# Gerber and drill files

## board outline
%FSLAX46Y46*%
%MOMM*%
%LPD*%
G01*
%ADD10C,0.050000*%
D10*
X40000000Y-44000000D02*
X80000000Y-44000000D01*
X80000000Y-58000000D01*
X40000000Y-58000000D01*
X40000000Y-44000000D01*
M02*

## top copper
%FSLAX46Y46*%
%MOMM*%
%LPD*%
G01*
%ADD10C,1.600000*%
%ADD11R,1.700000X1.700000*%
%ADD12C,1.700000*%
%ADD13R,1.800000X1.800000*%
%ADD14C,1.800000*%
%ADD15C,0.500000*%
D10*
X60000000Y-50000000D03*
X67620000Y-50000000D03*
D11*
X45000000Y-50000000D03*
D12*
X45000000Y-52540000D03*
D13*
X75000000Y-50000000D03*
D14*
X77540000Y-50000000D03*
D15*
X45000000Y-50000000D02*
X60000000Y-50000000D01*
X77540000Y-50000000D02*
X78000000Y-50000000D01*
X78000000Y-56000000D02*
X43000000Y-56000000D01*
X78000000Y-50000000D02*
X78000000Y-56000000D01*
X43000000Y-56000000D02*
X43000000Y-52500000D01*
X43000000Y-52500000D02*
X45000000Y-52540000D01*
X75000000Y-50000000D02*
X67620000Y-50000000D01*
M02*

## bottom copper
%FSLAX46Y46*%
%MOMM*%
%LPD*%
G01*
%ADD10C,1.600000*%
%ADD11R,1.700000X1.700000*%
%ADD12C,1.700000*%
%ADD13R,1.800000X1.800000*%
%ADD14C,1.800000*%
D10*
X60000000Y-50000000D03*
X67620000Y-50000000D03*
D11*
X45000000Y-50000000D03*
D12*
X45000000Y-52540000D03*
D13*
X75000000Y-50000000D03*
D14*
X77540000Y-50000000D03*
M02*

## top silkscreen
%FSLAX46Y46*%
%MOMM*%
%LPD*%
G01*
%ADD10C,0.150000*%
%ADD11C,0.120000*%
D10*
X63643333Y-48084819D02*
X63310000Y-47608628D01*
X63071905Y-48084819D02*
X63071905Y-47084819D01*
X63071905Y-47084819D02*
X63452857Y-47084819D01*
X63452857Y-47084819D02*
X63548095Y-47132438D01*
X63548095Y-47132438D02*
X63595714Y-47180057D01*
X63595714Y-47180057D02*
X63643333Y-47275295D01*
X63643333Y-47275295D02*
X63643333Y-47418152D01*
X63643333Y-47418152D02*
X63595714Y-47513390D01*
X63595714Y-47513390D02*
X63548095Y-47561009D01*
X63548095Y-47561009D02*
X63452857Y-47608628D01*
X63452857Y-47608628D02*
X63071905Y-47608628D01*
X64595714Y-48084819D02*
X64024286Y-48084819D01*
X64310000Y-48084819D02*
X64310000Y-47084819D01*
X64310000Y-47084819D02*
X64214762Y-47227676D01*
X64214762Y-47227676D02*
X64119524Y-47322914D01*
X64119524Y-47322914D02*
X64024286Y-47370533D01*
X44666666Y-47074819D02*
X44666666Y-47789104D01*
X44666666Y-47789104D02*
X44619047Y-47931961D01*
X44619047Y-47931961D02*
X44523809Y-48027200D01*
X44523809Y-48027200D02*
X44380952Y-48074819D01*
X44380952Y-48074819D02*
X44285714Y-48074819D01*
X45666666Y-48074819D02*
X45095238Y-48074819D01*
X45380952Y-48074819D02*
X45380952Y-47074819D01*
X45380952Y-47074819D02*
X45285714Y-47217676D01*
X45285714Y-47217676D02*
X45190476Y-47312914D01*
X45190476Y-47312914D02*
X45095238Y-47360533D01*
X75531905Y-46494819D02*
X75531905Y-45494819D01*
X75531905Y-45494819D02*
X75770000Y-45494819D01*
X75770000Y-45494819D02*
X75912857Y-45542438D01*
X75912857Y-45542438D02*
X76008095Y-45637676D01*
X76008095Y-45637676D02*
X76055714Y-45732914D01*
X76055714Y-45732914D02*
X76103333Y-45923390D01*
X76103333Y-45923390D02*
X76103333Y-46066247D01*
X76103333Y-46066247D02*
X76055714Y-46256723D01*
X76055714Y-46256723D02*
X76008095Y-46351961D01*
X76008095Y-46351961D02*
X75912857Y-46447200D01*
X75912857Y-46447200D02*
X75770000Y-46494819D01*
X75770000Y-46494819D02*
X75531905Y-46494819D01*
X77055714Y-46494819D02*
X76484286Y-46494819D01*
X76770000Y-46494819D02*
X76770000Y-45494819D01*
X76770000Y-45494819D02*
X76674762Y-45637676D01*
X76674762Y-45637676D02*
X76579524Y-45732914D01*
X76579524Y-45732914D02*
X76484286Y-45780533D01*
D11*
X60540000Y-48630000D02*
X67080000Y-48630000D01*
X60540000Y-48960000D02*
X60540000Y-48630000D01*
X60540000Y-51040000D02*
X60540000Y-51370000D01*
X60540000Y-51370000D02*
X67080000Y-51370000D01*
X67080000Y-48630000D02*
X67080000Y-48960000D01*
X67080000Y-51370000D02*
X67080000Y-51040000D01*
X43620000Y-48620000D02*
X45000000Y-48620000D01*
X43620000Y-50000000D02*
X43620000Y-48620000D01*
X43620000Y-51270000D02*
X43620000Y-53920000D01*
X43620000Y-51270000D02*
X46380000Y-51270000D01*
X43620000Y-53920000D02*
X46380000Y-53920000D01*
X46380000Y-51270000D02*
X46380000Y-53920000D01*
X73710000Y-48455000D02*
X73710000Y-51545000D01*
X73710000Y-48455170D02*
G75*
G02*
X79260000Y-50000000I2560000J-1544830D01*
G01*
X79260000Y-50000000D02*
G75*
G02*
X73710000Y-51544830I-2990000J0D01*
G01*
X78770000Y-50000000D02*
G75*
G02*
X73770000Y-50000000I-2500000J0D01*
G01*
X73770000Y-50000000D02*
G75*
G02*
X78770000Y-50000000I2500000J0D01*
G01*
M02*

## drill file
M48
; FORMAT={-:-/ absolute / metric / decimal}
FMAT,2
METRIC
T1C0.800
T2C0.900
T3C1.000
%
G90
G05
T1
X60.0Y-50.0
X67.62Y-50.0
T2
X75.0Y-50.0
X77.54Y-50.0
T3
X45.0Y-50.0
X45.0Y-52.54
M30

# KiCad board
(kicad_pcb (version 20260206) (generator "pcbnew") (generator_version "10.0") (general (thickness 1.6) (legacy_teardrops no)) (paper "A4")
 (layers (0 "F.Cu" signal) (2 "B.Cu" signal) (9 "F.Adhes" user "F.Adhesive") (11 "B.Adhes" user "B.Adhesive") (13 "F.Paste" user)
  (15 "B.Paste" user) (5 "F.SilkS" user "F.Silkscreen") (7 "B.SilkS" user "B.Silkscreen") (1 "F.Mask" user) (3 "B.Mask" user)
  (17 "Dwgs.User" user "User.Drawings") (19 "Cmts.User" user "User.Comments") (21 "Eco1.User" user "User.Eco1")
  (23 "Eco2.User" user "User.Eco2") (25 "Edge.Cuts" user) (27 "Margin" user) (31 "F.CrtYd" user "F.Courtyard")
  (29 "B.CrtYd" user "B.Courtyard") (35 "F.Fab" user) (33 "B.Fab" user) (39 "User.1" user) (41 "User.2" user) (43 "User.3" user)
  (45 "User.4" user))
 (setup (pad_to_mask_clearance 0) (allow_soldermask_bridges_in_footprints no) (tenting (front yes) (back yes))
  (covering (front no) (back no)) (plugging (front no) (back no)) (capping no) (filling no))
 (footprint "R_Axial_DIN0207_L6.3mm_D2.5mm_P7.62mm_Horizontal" (layer "F.Cu") (at 60 50)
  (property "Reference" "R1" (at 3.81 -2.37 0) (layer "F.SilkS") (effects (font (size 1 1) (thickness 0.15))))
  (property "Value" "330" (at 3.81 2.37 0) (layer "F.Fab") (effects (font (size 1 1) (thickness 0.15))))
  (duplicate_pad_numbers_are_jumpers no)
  (fp_line (start 0.54 -1.37) (end 7.08 -1.37) (stroke (width 0.12) (type solid)) (layer "F.SilkS"))
  (fp_line (start 0.54 -1.04) (end 0.54 -1.37) (stroke (width 0.12) (type solid)) (layer "F.SilkS"))
  (fp_line (start 0.54 1.04) (end 0.54 1.37) (stroke (width 0.12) (type solid)) (layer "F.SilkS"))
  (fp_line (start 0.54 1.37) (end 7.08 1.37) (stroke (width 0.12) (type solid)) (layer "F.SilkS"))
  (fp_line (start 7.08 -1.37) (end 7.08 -1.04) (stroke (width 0.12) (type solid)) (layer "F.SilkS"))
  (fp_line (start 7.08 1.37) (end 7.08 1.04) (stroke (width 0.12) (type solid)) (layer "F.SilkS"))
  (pad "1" thru_hole circle (at 0 0) (size 1.6 1.6) (drill 0.8) (layers "*.Cu" "*.Mask") (remove_unused_layers no) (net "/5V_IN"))
  (pad "2" thru_hole circle (at 7.62 0) (size 1.6 1.6) (drill 0.8) (layers "*.Cu" "*.Mask") (remove_unused_layers no) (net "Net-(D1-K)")))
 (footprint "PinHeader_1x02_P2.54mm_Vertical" (layer "F.Cu") (at 45 50)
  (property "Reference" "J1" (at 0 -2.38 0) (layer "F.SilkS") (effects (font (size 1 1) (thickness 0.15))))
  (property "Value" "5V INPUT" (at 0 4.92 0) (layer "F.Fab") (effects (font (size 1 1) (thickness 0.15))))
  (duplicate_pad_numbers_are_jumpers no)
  (fp_line (start -1.38 -1.38) (end 0 -1.38) (stroke (width 0.12) (type solid)) (layer "F.SilkS"))
  (fp_line (start -1.38 0) (end -1.38 -1.38) (stroke (width 0.12) (type solid)) (layer "F.SilkS"))
  (fp_line (start -1.38 1.27) (end -1.38 3.92) (stroke (width 0.12) (type solid)) (layer "F.SilkS"))
  (fp_line (start -1.38 1.27) (end 1.38 1.27) (stroke (width 0.12) (type solid)) (layer "F.SilkS"))
  (fp_line (start -1.38 3.92) (end 1.38 3.92) (stroke (width 0.12) (type solid)) (layer "F.SilkS"))
  (fp_line (start 1.38 1.27) (end 1.38 3.92) (stroke (width 0.12) (type solid)) (layer "F.SilkS"))
  (pad "1" thru_hole rect (at 0 0) (size 1.7 1.7) (drill 1) (layers "*.Cu" "*.Mask") (remove_unused_layers no) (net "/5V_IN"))
  (pad "2" thru_hole circle (at 0 2.54) (size 1.7 1.7) (drill 1) (layers "*.Cu" "*.Mask") (remove_unused_layers no) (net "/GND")))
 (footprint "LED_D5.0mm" (layer "F.Cu") (at 75 50)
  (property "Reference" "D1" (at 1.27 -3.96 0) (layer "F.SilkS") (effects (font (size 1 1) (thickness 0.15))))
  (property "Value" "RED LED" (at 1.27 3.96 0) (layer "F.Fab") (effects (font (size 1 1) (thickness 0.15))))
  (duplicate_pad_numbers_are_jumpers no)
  (fp_line (start -1.29 -1.545) (end -1.29 1.545) (stroke (width 0.12) (type solid)) (layer "F.SilkS"))
  (fp_arc (start -1.29 -1.54483) (mid 2.071779 -2.880495) (end 4.26 0) (stroke (width 0.12) (type solid)) (layer "F.SilkS"))
  (fp_arc (start 4.26 0) (mid 2.071779 2.880495) (end -1.29 1.54483) (stroke (width 0.12) (type solid)) (layer "F.SilkS"))
  (fp_circle (center 1.27 0) (end 3.77 0) (stroke (width 0.12) (type solid)) (fill no) (layer "F.SilkS"))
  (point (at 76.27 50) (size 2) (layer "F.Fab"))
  (pad "1" thru_hole rect (at 0 0) (size 1.8 1.8) (drill 0.9) (layers "*.Cu" "*.Mask") (remove_unused_layers no) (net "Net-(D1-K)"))
  (pad "2" thru_hole circle (at 2.54 0) (size 1.8 1.8) (drill 0.9) (layers "*.Cu" "*.Mask") (remove_unused_layers no) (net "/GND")))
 (gr_rect (start 40 44) (end 80 58) (stroke (width 0.05) (type default)) (fill no) (layer "Edge.Cuts"))
 (segment (start 45 50) (end 60 50) (width 0.5) (layer "F.Cu") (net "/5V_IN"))
 (segment (start 77.54 50) (end 78 50) (width 0.5) (layer "F.Cu") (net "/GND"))
 (segment (start 78 56) (end 43 56) (width 0.5) (layer "F.Cu") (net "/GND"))
 (segment (start 78 50) (end 78 56) (width 0.5) (layer "F.Cu") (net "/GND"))
 (segment (start 43 56) (end 43 52.5) (width 0.5) (layer "F.Cu") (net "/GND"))
 (segment (start 43 52.5) (end 45 52.54) (width 0.5) (layer "F.Cu") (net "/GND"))
 (segment (start 75 50) (end 67.62 50) (width 0.5) (layer "F.Cu") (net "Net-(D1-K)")))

